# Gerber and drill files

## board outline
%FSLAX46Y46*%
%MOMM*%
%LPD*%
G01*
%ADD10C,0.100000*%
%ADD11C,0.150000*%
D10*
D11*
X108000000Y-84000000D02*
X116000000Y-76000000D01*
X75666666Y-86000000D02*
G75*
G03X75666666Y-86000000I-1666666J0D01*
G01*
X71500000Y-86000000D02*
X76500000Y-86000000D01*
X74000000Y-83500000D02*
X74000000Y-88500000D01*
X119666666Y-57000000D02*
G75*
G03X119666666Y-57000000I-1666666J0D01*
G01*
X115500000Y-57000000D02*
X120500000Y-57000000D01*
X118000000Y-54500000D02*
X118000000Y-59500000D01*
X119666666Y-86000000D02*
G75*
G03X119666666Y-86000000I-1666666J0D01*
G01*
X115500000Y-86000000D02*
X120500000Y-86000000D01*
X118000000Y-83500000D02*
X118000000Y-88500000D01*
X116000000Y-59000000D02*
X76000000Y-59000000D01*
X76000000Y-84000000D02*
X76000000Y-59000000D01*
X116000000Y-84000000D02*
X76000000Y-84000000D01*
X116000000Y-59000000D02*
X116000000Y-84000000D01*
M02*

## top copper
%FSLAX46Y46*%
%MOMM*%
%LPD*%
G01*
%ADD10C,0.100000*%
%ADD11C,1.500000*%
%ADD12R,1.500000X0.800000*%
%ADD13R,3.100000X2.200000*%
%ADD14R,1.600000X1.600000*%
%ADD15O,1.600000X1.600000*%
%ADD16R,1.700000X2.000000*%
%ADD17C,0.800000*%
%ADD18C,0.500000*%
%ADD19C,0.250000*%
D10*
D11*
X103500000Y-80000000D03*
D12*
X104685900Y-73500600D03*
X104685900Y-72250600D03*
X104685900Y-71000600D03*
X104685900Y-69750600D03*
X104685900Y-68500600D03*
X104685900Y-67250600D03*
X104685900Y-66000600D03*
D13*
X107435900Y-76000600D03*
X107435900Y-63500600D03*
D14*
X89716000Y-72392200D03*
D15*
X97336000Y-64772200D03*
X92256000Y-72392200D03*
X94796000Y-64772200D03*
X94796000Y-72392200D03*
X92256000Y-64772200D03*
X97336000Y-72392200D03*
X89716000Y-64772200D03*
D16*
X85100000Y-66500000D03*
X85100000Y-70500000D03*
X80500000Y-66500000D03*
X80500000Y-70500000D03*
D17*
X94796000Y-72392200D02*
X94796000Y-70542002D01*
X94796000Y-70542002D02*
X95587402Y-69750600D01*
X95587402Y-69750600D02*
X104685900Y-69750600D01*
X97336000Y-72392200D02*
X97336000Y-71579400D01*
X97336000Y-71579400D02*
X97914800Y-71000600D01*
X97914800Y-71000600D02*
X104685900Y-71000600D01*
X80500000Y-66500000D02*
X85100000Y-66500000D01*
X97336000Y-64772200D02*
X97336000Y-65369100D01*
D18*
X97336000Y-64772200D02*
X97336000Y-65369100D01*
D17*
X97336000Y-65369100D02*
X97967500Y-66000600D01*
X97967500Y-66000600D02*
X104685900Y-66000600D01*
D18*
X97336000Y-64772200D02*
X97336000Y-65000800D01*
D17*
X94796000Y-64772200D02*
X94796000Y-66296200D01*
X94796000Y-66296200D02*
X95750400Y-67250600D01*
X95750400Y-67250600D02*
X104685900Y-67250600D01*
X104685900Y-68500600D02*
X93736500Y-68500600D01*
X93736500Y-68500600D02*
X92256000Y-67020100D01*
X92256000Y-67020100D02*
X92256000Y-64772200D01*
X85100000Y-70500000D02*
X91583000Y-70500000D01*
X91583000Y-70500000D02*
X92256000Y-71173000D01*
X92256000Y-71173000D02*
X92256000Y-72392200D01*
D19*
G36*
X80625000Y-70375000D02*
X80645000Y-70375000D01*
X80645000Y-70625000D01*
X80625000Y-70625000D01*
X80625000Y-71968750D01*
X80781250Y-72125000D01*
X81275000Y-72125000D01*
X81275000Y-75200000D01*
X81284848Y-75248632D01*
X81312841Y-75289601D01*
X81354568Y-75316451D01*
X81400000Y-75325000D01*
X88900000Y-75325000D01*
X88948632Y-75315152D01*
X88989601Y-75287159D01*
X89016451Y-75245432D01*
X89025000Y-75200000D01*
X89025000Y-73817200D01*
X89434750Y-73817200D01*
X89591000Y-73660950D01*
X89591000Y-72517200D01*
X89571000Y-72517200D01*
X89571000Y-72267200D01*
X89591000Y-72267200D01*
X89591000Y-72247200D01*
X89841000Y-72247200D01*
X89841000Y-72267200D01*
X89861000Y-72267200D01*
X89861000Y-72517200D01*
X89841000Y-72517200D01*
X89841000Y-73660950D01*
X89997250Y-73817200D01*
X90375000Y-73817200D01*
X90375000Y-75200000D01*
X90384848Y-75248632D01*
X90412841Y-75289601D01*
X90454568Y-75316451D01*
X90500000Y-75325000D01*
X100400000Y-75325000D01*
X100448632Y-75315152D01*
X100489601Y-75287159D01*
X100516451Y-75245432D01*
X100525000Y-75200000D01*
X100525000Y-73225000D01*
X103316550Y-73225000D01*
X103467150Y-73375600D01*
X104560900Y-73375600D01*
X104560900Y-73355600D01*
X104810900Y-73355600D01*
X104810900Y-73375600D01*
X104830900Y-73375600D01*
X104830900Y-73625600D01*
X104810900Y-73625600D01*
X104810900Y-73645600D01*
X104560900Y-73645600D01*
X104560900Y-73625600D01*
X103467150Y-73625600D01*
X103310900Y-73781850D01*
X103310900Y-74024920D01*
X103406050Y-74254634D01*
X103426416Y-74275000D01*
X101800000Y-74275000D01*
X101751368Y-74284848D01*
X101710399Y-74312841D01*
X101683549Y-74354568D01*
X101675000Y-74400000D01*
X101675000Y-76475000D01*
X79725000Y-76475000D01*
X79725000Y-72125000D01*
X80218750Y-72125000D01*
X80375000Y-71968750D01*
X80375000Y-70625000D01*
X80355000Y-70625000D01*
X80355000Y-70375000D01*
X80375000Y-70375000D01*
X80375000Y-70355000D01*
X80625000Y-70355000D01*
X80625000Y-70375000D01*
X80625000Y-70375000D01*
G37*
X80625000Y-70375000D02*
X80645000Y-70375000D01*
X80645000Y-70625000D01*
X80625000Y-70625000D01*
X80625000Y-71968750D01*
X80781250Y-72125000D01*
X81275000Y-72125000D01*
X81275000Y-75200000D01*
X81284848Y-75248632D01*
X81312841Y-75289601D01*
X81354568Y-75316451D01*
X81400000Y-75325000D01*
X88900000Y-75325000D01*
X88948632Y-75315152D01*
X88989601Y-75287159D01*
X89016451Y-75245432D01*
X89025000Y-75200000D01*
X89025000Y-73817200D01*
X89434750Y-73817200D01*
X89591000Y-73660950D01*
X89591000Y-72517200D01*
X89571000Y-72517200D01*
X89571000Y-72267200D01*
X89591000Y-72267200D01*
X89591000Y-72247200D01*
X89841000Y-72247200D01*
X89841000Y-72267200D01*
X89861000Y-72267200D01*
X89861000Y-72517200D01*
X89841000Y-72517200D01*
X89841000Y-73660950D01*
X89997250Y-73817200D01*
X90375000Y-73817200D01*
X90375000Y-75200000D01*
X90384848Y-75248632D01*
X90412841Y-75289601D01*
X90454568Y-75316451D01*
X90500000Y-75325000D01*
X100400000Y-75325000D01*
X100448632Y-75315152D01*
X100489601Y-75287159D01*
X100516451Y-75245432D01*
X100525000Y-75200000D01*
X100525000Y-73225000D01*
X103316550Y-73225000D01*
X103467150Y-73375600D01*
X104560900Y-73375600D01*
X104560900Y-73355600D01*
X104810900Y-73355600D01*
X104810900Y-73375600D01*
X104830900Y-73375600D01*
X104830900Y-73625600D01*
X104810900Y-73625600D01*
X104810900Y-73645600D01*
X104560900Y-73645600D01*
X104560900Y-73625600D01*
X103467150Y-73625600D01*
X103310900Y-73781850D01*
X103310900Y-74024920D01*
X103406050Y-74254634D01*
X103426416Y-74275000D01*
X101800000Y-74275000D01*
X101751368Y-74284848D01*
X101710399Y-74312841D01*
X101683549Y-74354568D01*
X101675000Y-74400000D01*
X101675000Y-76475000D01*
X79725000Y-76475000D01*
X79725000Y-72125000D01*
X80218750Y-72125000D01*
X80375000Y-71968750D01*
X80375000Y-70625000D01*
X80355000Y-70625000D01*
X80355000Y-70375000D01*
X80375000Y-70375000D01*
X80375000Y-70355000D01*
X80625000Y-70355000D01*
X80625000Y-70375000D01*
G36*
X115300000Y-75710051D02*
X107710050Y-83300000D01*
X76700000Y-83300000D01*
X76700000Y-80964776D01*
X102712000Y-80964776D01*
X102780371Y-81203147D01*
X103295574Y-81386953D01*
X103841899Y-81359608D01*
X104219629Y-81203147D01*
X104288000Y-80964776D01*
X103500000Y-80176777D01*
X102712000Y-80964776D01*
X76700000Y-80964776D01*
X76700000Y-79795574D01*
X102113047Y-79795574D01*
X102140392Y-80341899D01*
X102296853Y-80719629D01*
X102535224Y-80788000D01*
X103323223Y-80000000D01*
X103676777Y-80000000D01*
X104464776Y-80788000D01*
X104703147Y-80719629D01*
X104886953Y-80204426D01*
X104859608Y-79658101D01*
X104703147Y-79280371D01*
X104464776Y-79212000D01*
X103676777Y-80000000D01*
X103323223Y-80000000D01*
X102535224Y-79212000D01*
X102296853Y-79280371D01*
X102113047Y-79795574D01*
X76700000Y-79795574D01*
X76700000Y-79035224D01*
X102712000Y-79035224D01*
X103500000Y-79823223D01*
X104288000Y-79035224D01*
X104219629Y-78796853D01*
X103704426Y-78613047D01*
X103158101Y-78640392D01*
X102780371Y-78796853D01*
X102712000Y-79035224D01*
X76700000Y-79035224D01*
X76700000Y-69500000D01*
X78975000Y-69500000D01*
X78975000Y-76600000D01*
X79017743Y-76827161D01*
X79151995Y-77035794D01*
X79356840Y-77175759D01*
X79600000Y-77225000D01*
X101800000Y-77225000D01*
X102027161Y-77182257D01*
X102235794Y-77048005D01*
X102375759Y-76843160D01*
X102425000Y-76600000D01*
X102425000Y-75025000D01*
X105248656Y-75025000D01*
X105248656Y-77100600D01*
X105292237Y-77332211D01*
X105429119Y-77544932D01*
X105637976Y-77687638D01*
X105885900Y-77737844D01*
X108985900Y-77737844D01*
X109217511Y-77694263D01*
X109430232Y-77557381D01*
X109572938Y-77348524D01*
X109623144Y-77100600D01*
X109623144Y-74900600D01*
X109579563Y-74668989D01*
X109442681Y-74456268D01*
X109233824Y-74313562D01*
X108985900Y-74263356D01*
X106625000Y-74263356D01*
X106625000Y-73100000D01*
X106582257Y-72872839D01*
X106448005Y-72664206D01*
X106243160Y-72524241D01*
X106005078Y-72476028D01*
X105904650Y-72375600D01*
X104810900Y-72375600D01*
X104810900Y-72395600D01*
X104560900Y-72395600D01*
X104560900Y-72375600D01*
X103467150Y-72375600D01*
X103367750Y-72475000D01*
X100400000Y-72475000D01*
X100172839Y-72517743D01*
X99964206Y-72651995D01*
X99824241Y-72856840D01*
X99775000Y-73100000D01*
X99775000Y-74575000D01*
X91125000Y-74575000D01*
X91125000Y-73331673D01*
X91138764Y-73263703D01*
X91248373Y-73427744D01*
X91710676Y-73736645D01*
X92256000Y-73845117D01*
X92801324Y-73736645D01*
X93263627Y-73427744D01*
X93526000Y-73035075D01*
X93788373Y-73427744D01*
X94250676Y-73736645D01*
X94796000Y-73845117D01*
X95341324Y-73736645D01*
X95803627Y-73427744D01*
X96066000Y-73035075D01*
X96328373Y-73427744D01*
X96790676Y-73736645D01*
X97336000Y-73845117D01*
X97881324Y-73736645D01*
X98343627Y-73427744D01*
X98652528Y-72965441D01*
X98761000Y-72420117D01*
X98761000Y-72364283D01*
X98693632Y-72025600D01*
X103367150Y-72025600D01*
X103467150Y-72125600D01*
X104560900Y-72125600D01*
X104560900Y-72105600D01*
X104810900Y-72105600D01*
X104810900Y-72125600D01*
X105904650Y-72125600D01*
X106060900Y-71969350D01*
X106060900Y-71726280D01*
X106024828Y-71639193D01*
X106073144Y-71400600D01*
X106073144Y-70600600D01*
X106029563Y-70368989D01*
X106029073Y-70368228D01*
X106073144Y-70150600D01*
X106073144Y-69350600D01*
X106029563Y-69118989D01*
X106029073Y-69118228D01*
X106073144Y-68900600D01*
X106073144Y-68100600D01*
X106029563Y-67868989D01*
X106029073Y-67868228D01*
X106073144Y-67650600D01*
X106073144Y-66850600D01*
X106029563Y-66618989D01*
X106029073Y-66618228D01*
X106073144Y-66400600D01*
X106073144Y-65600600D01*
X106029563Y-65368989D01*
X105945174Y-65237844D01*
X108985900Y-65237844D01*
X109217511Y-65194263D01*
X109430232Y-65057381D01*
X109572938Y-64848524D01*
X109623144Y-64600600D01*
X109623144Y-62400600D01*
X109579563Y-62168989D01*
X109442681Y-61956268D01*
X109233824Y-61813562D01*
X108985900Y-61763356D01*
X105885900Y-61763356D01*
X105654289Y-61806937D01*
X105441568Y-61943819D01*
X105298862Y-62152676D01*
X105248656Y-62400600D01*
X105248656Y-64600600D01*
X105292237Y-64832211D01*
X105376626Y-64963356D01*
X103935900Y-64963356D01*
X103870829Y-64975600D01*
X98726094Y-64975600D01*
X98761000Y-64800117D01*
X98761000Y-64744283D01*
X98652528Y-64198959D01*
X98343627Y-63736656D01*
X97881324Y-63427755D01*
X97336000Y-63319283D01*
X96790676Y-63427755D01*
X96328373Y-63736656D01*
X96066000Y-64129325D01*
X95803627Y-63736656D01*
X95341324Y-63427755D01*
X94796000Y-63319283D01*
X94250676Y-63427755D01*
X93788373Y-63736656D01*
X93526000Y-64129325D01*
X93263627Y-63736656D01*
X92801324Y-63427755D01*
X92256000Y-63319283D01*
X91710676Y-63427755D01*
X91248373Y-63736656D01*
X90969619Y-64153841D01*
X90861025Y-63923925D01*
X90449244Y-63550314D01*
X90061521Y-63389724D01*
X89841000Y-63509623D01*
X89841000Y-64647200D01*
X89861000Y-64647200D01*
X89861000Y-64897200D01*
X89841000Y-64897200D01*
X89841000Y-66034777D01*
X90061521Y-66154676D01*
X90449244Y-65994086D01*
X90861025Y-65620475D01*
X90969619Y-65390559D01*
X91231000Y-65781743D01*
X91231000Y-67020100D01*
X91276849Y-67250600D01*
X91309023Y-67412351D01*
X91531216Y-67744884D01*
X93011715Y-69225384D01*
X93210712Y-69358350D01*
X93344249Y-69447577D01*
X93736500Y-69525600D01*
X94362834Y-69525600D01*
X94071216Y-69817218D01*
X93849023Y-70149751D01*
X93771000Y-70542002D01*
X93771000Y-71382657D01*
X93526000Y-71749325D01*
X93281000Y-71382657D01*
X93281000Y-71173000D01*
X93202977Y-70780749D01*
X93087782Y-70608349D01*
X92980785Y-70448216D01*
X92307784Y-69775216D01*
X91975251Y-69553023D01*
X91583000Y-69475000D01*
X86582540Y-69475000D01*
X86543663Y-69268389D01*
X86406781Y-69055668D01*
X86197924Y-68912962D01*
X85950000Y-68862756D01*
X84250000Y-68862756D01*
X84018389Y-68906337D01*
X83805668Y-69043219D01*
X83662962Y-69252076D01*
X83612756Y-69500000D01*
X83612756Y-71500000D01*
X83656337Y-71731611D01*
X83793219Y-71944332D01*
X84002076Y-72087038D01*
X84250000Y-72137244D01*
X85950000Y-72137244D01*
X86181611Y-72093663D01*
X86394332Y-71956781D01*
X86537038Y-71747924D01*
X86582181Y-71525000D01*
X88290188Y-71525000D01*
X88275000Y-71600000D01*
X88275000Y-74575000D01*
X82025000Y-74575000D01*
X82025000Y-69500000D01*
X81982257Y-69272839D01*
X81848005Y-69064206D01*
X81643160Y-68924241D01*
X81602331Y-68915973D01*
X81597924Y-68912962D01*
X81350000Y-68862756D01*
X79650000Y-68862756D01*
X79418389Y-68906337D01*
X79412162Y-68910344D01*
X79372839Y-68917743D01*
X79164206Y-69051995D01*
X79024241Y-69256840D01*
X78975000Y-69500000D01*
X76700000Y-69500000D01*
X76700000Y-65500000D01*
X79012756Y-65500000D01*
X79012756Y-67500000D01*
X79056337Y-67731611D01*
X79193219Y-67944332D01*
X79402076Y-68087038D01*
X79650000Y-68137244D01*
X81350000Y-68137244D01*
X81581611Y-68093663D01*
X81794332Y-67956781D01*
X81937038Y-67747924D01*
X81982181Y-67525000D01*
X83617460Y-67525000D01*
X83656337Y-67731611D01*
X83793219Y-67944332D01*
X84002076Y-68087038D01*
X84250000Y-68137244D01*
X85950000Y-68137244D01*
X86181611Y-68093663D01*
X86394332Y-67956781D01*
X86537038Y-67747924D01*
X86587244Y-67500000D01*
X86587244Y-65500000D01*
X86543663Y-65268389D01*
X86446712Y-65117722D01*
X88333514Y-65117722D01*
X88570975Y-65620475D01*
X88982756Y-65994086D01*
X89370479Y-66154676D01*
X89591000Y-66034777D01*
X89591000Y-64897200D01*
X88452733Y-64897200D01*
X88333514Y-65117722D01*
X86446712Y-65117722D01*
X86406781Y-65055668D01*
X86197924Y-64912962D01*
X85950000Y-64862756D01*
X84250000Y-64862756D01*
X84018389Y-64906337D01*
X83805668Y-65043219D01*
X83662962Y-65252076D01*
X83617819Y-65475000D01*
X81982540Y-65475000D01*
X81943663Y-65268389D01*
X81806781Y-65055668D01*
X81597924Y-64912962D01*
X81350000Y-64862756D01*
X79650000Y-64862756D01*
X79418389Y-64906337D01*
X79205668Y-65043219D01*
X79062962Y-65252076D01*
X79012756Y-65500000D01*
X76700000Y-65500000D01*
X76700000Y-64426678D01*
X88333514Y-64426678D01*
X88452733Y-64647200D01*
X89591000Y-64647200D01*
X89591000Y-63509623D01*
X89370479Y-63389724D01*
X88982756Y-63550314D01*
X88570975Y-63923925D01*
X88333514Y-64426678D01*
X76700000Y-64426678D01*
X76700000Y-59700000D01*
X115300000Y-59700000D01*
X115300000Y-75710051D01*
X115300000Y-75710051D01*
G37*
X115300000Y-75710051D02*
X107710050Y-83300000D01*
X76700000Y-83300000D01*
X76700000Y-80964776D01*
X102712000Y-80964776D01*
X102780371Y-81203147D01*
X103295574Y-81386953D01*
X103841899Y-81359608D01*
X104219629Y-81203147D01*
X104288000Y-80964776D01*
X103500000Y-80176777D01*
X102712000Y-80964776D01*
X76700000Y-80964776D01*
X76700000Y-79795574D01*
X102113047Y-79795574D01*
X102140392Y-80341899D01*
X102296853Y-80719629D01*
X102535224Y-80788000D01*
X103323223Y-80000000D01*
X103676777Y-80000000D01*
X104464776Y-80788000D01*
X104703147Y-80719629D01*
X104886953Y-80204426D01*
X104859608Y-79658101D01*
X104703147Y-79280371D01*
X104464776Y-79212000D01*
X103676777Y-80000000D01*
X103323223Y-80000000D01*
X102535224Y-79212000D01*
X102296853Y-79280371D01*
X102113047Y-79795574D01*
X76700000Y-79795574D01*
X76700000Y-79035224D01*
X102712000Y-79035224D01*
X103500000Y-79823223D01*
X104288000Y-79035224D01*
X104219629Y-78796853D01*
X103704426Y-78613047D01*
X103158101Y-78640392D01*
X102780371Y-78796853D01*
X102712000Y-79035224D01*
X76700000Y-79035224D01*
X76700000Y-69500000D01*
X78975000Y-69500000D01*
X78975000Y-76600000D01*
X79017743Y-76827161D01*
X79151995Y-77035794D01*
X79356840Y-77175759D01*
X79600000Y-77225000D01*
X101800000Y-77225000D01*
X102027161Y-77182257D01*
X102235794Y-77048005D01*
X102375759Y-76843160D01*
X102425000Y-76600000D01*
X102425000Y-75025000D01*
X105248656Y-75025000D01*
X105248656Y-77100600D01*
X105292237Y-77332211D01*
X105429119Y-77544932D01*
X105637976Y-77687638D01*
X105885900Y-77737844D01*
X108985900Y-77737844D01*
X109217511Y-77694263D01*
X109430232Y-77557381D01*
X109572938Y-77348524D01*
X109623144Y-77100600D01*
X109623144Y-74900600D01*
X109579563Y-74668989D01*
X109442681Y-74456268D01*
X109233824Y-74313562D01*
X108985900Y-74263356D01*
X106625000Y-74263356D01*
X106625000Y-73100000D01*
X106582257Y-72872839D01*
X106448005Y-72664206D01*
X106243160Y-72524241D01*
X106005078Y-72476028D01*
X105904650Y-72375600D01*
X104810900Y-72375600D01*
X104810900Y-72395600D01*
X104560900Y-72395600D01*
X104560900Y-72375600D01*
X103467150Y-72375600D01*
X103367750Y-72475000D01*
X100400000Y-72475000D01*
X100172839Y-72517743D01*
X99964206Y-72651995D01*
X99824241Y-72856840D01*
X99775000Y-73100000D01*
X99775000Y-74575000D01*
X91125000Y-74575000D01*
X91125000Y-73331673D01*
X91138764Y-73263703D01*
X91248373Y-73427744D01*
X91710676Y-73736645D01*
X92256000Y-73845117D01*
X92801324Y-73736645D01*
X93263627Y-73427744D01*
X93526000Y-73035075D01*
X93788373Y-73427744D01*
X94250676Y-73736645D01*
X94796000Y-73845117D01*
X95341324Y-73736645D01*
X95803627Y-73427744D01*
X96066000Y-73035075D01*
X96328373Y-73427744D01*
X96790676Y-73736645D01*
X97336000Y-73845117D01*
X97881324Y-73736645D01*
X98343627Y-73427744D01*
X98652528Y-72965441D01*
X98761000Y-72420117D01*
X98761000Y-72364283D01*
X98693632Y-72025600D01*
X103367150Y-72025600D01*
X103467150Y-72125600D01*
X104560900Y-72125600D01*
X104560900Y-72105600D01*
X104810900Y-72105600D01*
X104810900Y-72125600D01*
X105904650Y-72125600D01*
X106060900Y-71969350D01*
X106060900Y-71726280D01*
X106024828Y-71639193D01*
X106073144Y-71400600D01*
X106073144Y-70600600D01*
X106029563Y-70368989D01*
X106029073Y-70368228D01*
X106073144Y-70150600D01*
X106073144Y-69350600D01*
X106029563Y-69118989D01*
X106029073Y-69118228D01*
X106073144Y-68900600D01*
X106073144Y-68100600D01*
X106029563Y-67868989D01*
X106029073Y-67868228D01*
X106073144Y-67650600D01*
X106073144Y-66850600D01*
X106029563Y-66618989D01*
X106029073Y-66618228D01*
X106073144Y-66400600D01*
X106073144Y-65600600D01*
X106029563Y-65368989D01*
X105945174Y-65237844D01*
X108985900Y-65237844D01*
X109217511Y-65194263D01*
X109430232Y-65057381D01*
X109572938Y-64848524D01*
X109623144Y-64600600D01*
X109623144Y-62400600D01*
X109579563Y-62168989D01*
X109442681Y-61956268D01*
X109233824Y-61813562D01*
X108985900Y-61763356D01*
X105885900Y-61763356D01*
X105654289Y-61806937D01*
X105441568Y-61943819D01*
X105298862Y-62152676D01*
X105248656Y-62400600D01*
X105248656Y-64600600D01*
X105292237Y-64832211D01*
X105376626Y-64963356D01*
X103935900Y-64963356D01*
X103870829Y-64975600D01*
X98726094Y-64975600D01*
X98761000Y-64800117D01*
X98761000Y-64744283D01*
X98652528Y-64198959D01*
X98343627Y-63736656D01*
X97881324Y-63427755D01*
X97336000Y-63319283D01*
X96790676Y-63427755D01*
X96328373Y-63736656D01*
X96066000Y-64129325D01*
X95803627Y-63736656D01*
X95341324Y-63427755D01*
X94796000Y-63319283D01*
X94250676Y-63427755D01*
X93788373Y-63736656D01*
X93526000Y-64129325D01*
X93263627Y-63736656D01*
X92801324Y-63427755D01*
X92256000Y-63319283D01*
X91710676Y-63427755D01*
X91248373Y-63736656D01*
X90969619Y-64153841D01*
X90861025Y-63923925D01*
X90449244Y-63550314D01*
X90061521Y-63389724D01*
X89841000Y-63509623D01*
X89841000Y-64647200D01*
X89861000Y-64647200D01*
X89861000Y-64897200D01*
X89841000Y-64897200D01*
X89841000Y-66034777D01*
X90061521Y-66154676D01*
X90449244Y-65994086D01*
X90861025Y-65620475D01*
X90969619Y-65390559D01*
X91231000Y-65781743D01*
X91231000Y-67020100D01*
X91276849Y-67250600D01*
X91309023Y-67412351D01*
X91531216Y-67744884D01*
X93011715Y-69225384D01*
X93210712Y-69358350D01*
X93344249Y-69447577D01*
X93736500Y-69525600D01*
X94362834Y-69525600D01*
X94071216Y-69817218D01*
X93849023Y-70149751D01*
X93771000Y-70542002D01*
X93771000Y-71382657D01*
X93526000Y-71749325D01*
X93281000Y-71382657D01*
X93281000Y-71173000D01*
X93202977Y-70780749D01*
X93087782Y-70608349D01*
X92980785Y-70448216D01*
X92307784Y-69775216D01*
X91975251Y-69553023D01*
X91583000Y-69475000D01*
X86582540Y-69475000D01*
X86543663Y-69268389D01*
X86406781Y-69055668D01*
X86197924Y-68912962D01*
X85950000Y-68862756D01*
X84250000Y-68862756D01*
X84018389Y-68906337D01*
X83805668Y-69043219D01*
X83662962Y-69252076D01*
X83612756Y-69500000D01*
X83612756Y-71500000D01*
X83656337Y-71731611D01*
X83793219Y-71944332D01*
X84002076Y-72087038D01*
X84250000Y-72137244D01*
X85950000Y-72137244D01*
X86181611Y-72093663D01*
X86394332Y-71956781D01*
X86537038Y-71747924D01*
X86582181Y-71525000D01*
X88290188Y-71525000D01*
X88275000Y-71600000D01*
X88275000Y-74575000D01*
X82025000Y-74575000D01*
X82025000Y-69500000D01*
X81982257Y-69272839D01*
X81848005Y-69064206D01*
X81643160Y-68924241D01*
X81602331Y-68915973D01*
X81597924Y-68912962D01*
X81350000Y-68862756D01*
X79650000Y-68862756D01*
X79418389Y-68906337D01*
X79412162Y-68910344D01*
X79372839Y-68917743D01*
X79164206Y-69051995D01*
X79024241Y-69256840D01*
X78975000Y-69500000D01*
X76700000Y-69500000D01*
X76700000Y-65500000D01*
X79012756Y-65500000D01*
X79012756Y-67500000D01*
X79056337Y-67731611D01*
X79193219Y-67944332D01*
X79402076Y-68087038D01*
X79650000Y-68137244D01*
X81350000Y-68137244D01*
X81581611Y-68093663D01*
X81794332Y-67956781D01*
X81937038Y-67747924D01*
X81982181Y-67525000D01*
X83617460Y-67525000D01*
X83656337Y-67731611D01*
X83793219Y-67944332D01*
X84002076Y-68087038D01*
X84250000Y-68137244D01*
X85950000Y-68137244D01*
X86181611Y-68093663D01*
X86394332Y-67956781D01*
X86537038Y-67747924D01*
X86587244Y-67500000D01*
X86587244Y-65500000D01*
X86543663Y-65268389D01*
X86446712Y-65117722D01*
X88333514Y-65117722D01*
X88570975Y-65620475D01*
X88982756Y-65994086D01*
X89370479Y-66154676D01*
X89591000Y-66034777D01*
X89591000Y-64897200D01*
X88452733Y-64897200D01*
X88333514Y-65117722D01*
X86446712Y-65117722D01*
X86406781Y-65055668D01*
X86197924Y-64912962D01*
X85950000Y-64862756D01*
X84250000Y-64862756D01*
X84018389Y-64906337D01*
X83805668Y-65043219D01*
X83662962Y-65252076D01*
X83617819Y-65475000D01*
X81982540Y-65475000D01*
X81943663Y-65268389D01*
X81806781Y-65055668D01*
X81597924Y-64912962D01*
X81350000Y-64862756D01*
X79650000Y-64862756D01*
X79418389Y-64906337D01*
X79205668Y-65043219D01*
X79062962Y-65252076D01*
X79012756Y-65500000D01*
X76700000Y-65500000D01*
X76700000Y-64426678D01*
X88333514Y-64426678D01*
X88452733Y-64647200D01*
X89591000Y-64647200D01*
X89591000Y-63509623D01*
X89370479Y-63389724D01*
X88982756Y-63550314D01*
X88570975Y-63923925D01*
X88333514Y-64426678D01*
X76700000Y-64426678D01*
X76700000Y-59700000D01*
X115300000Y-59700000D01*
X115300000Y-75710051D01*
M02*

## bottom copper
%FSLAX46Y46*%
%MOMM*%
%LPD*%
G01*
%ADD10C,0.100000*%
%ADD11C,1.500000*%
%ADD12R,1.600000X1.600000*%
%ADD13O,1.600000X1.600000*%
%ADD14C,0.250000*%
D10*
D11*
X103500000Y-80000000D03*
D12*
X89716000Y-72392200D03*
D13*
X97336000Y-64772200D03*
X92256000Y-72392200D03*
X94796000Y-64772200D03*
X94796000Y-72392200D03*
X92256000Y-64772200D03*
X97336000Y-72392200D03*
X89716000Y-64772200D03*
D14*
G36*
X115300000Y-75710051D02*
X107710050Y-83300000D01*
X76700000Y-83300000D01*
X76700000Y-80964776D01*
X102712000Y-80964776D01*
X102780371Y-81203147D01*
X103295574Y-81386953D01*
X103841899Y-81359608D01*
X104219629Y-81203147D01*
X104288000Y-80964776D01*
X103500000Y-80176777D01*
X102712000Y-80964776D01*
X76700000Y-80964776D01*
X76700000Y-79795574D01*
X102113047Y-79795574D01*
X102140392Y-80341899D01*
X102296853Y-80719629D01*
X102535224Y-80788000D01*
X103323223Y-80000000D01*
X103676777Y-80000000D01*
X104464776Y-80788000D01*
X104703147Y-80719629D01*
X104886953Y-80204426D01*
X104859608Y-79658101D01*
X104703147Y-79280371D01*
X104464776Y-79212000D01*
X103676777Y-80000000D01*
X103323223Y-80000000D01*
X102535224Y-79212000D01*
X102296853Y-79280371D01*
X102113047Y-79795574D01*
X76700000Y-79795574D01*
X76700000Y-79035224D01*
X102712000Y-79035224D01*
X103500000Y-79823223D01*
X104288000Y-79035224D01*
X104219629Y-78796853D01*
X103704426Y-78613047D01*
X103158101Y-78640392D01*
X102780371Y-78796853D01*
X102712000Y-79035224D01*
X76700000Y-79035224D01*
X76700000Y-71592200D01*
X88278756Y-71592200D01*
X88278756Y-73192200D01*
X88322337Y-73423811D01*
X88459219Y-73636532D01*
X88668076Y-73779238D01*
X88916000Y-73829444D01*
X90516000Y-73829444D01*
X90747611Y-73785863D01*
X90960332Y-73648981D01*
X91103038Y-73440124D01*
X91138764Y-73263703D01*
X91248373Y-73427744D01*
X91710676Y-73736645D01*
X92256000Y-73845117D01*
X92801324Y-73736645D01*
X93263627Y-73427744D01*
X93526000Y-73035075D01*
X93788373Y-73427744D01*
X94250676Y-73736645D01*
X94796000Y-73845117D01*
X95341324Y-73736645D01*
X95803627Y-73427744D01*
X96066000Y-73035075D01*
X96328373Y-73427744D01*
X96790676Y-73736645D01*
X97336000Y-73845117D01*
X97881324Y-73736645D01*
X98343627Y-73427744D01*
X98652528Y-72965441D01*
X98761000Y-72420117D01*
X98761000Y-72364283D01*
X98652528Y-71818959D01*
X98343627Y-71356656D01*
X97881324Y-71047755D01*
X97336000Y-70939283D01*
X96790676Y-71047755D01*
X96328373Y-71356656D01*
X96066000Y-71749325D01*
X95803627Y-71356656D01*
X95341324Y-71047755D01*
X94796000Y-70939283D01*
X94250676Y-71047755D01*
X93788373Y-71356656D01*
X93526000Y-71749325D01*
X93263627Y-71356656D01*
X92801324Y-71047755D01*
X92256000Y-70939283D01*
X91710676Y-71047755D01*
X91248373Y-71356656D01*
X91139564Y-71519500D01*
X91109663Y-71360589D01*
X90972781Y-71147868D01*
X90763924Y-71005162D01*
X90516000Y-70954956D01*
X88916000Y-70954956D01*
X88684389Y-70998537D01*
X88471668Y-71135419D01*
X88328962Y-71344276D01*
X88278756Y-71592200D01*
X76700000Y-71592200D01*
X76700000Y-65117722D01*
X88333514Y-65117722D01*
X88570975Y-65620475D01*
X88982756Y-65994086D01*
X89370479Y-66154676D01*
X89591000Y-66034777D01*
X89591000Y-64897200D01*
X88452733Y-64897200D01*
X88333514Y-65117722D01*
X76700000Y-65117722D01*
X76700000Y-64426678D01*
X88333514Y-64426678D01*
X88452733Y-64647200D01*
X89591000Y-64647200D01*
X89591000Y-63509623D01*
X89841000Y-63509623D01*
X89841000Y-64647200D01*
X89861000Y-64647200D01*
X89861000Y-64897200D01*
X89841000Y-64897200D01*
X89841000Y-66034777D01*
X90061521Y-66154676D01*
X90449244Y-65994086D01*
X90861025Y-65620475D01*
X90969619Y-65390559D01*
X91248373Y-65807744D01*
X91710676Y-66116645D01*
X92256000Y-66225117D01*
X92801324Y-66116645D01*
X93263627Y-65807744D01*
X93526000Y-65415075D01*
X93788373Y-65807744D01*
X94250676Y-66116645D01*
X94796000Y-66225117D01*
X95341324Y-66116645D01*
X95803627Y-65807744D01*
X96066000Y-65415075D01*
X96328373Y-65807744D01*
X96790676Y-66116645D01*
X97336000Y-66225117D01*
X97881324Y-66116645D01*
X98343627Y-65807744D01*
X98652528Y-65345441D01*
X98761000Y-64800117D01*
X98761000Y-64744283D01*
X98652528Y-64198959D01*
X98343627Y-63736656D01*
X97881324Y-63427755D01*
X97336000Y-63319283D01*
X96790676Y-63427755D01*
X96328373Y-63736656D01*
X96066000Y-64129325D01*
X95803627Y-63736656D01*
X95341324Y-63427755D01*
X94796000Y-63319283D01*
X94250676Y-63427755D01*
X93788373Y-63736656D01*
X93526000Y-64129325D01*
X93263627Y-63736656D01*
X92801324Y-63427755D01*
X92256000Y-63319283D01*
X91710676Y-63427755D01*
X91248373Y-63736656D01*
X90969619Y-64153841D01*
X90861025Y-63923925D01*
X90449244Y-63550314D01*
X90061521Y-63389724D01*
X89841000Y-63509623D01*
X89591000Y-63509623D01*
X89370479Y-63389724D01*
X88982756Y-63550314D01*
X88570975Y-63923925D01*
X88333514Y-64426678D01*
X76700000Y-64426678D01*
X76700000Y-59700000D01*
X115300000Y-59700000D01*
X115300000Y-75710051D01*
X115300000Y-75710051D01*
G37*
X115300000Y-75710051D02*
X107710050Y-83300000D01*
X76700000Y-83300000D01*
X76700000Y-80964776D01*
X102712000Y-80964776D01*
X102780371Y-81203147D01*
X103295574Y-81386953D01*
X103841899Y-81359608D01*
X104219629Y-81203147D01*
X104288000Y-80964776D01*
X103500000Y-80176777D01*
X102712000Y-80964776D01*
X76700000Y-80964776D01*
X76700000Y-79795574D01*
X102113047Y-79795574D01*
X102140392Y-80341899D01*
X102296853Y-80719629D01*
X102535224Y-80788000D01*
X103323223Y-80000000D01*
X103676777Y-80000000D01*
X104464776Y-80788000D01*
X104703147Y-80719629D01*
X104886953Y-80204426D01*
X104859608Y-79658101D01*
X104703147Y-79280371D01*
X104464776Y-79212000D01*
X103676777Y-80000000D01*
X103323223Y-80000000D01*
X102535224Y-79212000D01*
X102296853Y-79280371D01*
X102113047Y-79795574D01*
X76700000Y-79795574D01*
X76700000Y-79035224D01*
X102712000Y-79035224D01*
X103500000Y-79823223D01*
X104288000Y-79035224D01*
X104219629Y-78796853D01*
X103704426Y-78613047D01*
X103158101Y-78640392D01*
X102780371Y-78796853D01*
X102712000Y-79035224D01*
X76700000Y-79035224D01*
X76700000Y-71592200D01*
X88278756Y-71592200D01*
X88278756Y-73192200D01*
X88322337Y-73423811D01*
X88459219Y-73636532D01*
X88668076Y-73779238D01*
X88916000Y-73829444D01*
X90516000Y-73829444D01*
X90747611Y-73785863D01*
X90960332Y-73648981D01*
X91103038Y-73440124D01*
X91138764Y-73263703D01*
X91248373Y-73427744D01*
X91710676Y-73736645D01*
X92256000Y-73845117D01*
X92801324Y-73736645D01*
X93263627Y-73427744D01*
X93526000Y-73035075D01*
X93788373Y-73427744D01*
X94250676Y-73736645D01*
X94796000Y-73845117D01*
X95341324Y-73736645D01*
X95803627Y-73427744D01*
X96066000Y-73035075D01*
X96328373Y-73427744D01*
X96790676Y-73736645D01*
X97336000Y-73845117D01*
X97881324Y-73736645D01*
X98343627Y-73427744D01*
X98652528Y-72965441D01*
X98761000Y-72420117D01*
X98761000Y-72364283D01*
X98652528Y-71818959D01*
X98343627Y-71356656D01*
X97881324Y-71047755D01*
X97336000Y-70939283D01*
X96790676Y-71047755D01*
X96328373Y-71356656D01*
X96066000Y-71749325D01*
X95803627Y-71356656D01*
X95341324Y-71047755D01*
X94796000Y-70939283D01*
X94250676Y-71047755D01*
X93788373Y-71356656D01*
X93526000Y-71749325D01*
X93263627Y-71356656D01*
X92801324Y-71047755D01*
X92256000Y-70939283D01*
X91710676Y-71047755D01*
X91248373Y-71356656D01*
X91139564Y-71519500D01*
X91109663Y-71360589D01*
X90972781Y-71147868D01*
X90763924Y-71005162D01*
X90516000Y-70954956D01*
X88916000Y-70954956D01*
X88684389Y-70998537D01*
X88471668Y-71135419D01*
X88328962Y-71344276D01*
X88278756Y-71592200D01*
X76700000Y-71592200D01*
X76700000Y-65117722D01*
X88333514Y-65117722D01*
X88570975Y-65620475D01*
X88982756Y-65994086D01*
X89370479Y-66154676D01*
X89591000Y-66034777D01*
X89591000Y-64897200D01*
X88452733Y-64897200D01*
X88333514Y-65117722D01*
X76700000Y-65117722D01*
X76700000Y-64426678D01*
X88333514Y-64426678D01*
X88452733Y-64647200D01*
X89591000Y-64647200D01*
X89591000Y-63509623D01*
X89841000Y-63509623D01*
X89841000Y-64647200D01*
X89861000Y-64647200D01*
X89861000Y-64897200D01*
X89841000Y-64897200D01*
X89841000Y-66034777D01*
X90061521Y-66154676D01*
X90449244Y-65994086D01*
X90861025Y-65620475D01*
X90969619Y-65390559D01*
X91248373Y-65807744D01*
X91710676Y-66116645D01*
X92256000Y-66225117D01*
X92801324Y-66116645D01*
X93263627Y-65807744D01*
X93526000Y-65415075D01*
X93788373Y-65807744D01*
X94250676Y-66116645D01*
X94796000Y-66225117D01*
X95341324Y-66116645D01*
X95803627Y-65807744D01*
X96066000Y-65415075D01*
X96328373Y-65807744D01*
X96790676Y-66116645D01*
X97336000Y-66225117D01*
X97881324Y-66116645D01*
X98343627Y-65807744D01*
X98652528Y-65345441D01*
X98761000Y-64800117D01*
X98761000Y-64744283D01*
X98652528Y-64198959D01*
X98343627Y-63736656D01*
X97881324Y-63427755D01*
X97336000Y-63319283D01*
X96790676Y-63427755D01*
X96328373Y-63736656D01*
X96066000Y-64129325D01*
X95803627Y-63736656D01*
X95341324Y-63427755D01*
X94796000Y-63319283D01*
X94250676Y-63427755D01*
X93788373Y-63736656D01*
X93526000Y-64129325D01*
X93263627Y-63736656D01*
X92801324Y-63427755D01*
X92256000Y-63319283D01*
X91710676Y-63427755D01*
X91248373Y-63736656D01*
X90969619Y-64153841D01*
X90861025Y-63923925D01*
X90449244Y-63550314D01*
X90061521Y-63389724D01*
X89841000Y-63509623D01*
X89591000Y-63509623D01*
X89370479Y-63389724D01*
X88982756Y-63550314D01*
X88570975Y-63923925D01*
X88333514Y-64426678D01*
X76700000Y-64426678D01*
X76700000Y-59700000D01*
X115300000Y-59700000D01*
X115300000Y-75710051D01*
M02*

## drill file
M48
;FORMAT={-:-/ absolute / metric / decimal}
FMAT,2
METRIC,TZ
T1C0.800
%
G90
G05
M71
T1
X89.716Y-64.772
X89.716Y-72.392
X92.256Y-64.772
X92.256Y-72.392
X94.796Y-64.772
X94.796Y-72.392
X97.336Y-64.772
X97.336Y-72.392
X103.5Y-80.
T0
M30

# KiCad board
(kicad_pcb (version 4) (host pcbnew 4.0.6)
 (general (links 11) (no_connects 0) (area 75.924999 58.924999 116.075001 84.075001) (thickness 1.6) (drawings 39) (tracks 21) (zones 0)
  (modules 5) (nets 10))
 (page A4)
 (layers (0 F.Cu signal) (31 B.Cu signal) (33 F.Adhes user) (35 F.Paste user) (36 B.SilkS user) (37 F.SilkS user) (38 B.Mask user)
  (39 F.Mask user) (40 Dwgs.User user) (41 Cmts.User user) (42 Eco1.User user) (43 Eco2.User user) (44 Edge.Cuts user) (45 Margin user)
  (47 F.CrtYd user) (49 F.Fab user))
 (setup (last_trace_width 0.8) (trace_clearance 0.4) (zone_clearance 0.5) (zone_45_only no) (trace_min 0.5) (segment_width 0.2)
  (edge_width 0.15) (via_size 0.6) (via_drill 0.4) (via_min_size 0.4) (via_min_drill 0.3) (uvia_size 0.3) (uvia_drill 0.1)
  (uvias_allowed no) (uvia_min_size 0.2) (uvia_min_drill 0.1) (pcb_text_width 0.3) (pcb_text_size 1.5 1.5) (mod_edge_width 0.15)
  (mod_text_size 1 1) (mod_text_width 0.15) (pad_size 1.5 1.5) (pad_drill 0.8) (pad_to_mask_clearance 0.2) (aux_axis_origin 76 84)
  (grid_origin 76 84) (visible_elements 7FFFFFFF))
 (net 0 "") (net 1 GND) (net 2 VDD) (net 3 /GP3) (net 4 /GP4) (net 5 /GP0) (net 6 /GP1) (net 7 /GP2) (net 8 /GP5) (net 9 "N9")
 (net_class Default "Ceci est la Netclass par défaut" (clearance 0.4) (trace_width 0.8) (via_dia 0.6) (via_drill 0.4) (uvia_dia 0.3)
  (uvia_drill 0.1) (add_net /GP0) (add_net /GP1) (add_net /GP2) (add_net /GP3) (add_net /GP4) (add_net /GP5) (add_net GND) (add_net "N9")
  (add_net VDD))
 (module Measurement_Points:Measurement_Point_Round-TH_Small (layer F.Cu) (at 103.5 80)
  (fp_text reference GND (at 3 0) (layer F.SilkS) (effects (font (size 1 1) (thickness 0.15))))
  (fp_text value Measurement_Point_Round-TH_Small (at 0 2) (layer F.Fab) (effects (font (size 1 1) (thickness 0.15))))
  (pad 1 thru_hole circle (at 0 0) (size 1.5 1.5) (drill 0.8) (layers *.Cu *.Mask) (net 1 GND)))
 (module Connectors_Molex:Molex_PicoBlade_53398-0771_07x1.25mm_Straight (layer F.Cu) (at 106.0609 69.7506 90)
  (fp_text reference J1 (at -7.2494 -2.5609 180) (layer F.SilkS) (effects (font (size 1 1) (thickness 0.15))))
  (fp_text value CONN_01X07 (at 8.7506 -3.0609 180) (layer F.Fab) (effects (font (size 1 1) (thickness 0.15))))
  (pad 1 smd rect (at -3.75 -1.375 90) (size 0.8 1.5) (layers F.Cu F.Paste F.Mask) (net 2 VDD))
  (pad 2 smd rect (at -2.5 -1.375 90) (size 0.8 1.5) (layers F.Cu F.Paste F.Mask) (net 1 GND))
  (pad 3 smd rect (at -1.25 -1.375 90) (size 0.8 1.5) (layers F.Cu F.Paste F.Mask) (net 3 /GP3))
  (pad 4 smd rect (at 0 -1.375 90) (size 0.8 1.5) (layers F.Cu F.Paste F.Mask) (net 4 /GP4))
  (pad 5 smd rect (at 1.25 -1.375 90) (size 0.8 1.5) (layers F.Cu F.Paste F.Mask) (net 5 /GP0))
  (pad 6 smd rect (at 2.5 -1.375 90) (size 0.8 1.5) (layers F.Cu F.Paste F.Mask) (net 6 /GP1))
  (pad 7 smd rect (at 3.75 -1.375 90) (size 0.8 1.5) (layers F.Cu F.Paste F.Mask) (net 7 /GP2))
  (pad "" smd rect (at -6.25 1.375 90) (size 2.2 3.1) (layers F.Cu F.Paste F.Mask))
  (pad "" smd rect (at 6.25 1.375 90) (size 2.2 3.1) (layers F.Cu F.Paste F.Mask)))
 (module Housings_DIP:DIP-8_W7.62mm (layer F.Cu) (at 89.716 72.3922 90)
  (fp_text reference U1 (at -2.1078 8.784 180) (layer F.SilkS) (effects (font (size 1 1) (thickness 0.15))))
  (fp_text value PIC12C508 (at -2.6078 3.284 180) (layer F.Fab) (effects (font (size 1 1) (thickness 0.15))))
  (pad 1 thru_hole rect (at 0 0 90) (size 1.6 1.6) (drill 0.8) (layers *.Cu *.Mask) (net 2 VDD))
  (pad 5 thru_hole oval (at 7.62 7.62 90) (size 1.6 1.6) (drill 0.8) (layers *.Cu *.Mask) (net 7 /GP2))
  (pad 2 thru_hole oval (at 0 2.54 90) (size 1.6 1.6) (drill 0.8) (layers *.Cu *.Mask) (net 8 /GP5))
  (pad 6 thru_hole oval (at 7.62 5.08 90) (size 1.6 1.6) (drill 0.8) (layers *.Cu *.Mask) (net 6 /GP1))
  (pad 3 thru_hole oval (at 0 5.08 90) (size 1.6 1.6) (drill 0.8) (layers *.Cu *.Mask) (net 4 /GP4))
  (pad 7 thru_hole oval (at 7.62 2.54 90) (size 1.6 1.6) (drill 0.8) (layers *.Cu *.Mask) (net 5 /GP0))
  (pad 4 thru_hole oval (at 0 7.62 90) (size 1.6 1.6) (drill 0.8) (layers *.Cu *.Mask) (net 3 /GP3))
  (pad 8 thru_hole oval (at 7.62 0 90) (size 1.6 1.6) (drill 0.8) (layers *.Cu *.Mask) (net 1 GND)))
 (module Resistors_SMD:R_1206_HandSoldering (layer F.Cu) (at 85.1 68.5 270)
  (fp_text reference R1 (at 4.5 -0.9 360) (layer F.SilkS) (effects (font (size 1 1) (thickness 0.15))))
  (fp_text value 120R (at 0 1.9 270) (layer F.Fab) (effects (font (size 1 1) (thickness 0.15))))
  (pad 1 smd rect (at -2 0 270) (size 2 1.7) (layers F.Cu F.Paste F.Mask) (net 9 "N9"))
  (pad 2 smd rect (at 2 0 270) (size 2 1.7) (layers F.Cu F.Paste F.Mask) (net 8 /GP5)))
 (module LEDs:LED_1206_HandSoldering (layer F.Cu) (at 80.5 68.5 270)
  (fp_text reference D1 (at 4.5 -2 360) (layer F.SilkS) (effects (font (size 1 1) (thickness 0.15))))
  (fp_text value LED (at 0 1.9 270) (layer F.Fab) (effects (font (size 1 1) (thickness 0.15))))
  (pad 1 smd rect (at -2 0 270) (size 2 1.7) (layers F.Cu F.Paste F.Mask) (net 9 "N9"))
  (pad 2 smd rect (at 2 0 270) (size 2 1.7) (layers F.Cu F.Paste F.Mask) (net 2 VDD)))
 (gr_line (start 108 84) (end 116 76) (angle 90) (layer Edge.Cuts) (width 0.15))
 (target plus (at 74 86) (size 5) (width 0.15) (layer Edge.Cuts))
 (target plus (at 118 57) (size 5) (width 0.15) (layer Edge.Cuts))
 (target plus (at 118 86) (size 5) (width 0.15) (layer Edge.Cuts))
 (gr_line (start 116 59) (end 76 59) (angle 90) (layer Edge.Cuts) (width 0.15))
 (gr_line (start 76 84) (end 76 59) (angle 90) (layer Edge.Cuts) (width 0.15))
 (gr_line (start 116 84) (end 76 84) (angle 90) (layer Edge.Cuts) (width 0.15))
 (gr_line (start 116 59) (end 116 84) (angle 90) (layer Edge.Cuts) (width 0.15))
 (segment (start 94.796 72.3922) (end 94.796 70.542002) (width 0.8) (layer F.Cu) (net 4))
 (segment (start 94.796 70.542002) (end 95.587402 69.7506) (width 0.8) (layer F.Cu) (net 4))
 (segment (start 95.587402 69.7506) (end 104.6859 69.7506) (width 0.8) (layer F.Cu) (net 4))
 (segment (start 97.336 72.3922) (end 97.336 71.5794) (width 0.8) (layer F.Cu) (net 3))
 (segment (start 97.336 71.5794) (end 97.9148 71.0006) (width 0.8) (layer F.Cu) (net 3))
 (segment (start 97.9148 71.0006) (end 104.6859 71.0006) (width 0.8) (layer F.Cu) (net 3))
 (segment (start 80.5 66.5) (end 85.1 66.5) (width 0.8) (layer F.Cu) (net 9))
 (segment (start 97.336 64.7722) (end 97.336 65.3691) (width 0.8) (layer F.Cu) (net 7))
 (segment (start 97.336 64.7722) (end 97.336 65.3691) (width 0.5) (layer F.Cu) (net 7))
 (segment (start 97.336 65.3691) (end 97.9675 66.0006) (width 0.8) (layer F.Cu) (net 7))
 (segment (start 97.9675 66.0006) (end 104.6859 66.0006) (width 0.8) (layer F.Cu) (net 7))
 (segment (start 97.336 64.7722) (end 97.336 65.0008) (width 0.5) (layer F.Cu) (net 7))
 (segment (start 94.796 64.7722) (end 94.796 66.2962) (width 0.8) (layer F.Cu) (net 6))
 (segment (start 94.796 66.2962) (end 95.7504 67.2506) (width 0.8) (layer F.Cu) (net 6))
 (segment (start 95.7504 67.2506) (end 104.6859 67.2506) (width 0.8) (layer F.Cu) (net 6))
 (segment (start 104.6859 68.5006) (end 93.7365 68.5006) (width 0.8) (layer F.Cu) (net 5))
 (segment (start 93.7365 68.5006) (end 92.256 67.0201) (width 0.8) (layer F.Cu) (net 5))
 (segment (start 92.256 67.0201) (end 92.256 64.7722) (width 0.8) (layer F.Cu) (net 5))
 (segment (start 85.1 70.5) (end 91.583 70.5) (width 0.8) (layer F.Cu) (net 8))
 (segment (start 91.583 70.5) (end 92.256 71.173) (width 0.8) (layer F.Cu) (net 8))
 (segment (start 92.256 71.173) (end 92.256 72.3922) (width 0.8) (layer F.Cu) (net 8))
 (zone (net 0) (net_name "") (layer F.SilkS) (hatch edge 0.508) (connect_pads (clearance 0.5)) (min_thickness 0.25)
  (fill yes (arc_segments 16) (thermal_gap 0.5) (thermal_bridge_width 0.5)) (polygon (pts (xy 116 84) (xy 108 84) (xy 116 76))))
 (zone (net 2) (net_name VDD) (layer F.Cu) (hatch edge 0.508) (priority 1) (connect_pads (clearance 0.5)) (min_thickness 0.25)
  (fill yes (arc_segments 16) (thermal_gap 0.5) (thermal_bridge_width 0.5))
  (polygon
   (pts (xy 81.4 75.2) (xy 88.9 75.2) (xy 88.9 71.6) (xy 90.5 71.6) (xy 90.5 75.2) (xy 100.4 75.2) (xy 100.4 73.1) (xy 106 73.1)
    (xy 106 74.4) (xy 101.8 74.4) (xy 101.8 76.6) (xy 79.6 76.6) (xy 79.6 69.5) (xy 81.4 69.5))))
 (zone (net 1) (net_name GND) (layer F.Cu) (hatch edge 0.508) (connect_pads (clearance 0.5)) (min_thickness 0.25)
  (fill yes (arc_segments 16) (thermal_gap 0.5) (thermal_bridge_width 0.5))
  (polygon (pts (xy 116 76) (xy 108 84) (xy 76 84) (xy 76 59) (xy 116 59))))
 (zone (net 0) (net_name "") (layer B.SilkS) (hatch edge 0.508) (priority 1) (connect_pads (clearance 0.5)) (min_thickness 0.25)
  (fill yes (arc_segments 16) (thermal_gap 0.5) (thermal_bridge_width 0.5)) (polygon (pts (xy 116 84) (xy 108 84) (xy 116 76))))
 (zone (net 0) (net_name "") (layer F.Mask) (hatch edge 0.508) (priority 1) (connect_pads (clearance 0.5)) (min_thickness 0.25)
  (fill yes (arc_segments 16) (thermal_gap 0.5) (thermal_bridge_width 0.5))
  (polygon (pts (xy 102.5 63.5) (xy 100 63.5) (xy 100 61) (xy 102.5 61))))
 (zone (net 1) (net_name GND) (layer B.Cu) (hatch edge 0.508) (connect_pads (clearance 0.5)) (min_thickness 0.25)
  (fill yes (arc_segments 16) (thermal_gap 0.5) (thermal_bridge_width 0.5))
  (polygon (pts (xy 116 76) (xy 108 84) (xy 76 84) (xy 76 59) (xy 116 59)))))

